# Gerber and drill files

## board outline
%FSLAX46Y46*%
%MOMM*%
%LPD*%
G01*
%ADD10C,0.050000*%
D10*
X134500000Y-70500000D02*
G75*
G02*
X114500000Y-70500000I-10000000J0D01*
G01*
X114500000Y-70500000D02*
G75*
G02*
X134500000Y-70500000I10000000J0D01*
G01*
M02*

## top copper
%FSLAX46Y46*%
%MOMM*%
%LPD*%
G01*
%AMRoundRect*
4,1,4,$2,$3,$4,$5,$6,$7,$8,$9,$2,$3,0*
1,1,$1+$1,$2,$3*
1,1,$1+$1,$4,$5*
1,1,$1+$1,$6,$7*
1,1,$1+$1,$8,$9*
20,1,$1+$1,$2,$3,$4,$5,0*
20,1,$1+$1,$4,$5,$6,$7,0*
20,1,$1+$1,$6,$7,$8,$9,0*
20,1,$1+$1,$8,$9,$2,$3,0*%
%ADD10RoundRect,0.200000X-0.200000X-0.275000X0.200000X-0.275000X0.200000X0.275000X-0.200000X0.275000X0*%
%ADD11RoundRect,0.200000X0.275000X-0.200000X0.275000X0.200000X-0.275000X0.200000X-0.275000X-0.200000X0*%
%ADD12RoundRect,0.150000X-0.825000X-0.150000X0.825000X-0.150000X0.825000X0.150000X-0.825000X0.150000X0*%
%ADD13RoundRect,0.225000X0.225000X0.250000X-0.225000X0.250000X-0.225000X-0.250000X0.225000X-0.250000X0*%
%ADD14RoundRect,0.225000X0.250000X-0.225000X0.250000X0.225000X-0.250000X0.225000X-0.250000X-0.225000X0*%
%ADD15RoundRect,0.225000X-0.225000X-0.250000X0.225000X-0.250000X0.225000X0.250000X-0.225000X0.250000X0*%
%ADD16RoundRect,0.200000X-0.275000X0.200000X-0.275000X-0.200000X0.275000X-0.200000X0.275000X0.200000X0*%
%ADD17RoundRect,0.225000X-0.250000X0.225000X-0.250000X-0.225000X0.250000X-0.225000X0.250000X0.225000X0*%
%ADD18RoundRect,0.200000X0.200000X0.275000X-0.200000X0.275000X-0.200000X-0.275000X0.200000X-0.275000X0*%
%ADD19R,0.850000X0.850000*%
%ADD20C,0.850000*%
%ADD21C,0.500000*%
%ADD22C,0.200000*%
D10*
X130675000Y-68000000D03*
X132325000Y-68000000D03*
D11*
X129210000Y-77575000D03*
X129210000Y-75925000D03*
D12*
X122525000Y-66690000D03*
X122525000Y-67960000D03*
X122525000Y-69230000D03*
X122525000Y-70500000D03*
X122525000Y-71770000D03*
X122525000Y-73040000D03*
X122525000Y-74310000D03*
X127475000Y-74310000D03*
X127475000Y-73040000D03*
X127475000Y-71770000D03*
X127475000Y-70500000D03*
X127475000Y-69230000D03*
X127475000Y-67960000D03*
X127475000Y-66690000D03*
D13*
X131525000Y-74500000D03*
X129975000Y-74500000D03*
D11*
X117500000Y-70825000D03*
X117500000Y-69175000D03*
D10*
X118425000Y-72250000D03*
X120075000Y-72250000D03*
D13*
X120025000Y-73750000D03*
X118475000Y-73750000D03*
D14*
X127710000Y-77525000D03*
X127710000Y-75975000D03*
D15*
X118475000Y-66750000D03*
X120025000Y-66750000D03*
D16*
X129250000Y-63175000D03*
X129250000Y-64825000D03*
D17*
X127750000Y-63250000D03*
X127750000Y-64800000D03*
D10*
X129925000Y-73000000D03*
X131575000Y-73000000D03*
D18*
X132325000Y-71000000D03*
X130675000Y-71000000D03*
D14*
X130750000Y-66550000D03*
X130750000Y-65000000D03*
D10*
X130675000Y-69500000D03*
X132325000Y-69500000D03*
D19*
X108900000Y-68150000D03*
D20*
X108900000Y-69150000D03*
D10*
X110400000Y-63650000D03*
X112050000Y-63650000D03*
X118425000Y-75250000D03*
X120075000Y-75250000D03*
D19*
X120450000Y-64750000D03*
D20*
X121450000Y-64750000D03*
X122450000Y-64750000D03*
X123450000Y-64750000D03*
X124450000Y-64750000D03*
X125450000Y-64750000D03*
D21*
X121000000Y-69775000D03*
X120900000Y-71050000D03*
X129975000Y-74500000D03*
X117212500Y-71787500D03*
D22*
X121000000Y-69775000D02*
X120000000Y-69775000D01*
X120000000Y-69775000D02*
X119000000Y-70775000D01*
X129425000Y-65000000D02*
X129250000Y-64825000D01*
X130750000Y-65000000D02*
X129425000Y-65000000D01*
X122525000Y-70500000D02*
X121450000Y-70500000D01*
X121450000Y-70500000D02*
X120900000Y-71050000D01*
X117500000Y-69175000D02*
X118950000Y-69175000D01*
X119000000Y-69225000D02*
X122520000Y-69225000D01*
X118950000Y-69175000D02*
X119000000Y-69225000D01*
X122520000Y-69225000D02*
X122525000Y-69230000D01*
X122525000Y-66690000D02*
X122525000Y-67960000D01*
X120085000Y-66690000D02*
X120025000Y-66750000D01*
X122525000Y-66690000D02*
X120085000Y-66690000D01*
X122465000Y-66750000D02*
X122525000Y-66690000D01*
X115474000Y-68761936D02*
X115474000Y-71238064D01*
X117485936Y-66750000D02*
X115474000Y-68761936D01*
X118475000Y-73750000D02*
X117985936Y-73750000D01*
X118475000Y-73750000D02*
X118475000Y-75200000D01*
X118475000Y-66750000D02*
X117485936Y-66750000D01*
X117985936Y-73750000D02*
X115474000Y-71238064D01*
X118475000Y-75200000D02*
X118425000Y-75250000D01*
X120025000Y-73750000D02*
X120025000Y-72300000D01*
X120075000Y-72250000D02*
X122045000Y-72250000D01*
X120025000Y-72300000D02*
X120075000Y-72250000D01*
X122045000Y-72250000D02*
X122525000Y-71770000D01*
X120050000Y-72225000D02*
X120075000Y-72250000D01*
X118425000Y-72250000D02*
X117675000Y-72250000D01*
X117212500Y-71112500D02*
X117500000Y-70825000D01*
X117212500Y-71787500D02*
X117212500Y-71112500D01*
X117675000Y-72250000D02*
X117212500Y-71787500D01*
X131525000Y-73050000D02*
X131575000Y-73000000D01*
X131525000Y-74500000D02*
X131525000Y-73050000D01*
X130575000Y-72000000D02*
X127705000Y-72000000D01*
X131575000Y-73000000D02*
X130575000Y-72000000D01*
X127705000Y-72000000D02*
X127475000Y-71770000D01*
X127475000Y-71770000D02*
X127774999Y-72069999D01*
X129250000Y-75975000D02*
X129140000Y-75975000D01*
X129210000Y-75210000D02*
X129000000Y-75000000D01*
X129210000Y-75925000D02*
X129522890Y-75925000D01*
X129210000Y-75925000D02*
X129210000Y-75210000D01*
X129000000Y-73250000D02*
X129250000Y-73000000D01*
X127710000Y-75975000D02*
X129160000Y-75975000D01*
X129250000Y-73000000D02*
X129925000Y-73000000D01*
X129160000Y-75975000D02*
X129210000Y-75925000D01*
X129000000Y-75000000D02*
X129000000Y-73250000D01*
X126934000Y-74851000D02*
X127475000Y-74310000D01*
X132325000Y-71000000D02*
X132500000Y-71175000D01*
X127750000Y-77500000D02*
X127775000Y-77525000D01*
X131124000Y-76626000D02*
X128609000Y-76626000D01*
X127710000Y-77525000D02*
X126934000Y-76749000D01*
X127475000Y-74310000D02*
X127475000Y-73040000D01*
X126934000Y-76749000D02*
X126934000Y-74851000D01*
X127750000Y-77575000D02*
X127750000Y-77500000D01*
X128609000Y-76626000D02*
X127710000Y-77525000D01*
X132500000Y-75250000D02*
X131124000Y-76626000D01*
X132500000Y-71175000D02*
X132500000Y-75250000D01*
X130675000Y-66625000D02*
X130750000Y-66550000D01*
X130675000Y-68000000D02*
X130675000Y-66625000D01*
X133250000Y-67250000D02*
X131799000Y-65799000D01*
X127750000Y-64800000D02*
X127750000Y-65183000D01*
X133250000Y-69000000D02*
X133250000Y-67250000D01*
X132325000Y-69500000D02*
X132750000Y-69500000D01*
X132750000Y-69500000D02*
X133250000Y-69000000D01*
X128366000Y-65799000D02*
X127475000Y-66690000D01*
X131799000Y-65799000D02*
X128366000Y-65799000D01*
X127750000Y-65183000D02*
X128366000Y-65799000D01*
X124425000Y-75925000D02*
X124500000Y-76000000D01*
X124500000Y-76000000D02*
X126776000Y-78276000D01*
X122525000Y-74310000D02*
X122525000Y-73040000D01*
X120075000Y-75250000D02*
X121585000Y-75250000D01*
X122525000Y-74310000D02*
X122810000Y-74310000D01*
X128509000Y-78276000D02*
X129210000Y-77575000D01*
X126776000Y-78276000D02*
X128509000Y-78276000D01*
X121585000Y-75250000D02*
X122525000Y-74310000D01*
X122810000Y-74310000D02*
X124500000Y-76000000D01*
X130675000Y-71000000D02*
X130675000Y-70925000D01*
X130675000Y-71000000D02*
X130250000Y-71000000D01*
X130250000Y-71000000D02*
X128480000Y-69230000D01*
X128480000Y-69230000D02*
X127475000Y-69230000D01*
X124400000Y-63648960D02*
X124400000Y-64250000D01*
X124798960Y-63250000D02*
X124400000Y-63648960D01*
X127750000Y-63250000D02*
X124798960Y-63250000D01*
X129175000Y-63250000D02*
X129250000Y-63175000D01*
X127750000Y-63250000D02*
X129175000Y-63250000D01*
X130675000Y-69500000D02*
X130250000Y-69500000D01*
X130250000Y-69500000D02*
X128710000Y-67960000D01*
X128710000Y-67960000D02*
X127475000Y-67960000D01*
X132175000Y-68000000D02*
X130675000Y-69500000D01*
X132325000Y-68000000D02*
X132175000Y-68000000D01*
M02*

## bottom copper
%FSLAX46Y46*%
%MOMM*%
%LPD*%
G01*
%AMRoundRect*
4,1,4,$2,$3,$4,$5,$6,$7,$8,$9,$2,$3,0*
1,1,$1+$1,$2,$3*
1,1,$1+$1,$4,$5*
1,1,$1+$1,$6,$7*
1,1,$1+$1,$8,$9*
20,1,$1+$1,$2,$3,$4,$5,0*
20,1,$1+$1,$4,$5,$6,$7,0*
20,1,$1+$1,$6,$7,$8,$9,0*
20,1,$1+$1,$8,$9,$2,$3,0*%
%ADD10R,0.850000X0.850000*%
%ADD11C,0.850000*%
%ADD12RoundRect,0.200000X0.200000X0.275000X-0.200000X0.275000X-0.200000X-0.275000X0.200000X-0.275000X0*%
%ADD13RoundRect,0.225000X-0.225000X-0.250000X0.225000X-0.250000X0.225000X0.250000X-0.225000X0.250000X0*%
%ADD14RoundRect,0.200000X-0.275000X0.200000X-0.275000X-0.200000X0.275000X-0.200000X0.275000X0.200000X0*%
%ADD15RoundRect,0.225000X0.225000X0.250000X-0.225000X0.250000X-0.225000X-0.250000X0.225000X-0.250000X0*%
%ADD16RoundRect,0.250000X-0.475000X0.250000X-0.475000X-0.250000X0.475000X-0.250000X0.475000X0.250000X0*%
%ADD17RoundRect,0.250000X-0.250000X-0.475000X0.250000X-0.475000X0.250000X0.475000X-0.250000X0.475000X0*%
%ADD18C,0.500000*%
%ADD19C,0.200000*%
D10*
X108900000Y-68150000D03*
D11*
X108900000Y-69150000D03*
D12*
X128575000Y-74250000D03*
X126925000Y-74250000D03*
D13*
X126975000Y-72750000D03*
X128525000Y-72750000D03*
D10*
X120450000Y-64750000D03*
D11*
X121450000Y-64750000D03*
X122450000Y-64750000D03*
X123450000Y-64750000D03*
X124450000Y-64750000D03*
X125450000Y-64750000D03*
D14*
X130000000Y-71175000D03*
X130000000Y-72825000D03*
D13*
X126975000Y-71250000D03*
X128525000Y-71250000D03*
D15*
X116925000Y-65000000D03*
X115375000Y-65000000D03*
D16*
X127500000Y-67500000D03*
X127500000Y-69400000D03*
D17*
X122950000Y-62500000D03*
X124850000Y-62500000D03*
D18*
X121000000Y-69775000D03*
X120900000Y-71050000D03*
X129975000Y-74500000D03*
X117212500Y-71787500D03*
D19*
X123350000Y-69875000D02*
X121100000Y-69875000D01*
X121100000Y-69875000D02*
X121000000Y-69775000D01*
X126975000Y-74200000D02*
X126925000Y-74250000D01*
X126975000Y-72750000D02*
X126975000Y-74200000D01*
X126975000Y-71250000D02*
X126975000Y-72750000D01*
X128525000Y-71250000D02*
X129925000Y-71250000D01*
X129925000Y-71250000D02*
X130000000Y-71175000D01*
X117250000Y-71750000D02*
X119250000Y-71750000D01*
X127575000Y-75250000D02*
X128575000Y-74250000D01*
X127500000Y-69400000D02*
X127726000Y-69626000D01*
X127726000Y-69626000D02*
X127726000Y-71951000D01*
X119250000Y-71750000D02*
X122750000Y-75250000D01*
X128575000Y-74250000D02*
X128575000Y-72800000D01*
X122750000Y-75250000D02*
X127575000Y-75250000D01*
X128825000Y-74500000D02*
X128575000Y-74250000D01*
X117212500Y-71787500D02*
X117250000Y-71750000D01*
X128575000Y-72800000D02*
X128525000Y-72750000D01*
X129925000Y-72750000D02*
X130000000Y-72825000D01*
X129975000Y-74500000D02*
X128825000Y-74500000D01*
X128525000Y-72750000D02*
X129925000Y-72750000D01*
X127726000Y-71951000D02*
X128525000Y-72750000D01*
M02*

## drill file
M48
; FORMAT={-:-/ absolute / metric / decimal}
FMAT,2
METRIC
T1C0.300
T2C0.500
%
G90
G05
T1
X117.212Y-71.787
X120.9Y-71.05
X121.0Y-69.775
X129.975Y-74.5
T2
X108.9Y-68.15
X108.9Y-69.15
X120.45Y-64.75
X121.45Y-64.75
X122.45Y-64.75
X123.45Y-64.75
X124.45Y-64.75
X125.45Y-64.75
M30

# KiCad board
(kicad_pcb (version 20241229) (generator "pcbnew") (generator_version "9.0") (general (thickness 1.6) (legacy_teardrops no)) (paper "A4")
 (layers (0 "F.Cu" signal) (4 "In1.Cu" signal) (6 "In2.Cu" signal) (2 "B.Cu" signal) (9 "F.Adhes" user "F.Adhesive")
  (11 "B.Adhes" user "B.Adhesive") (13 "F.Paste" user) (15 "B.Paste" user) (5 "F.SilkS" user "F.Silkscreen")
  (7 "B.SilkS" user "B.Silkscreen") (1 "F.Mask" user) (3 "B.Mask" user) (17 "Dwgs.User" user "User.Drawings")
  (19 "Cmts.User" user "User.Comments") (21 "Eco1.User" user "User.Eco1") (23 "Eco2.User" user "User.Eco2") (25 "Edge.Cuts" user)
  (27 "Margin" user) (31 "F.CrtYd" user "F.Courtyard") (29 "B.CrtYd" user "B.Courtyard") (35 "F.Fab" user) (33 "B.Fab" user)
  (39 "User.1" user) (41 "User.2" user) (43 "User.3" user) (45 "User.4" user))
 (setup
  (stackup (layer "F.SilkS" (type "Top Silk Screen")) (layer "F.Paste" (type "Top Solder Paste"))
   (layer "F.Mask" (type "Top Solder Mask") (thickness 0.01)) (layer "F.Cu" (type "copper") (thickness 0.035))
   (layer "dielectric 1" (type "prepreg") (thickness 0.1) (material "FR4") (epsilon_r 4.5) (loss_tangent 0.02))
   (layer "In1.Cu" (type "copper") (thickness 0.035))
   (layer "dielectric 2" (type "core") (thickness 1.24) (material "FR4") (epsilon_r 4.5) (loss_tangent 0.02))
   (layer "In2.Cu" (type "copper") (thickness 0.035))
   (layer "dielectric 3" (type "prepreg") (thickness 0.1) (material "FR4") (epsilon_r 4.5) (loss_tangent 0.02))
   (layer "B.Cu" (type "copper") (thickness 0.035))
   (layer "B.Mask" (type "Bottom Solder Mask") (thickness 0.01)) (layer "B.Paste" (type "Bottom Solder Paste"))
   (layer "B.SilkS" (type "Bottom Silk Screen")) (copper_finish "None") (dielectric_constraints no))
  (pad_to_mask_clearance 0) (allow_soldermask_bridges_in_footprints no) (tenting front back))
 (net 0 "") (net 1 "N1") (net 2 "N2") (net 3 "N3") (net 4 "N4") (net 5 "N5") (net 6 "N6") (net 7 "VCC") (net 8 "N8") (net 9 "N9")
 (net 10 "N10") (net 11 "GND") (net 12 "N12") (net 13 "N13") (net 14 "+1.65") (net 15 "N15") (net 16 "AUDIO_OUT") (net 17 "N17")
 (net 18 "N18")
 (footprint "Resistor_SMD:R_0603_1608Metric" (layer "F.Cu") (at 131.5 68)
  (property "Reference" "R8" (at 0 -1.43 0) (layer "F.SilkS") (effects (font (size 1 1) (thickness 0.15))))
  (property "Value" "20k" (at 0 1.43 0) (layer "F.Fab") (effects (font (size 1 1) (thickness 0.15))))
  (pad "1" smd roundrect (at -0.825 0) (size 0.8 0.95) (layers "F.Cu" "F.Mask" "F.Paste") (roundrect_rratio 0.25) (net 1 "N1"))
  (pad "2" smd roundrect (at 0.825 0) (size 0.8 0.95) (layers "F.Cu" "F.Mask" "F.Paste") (roundrect_rratio 0.25) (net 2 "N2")))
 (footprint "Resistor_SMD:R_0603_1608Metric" (layer "F.Cu") (at 129.21 76.75 90)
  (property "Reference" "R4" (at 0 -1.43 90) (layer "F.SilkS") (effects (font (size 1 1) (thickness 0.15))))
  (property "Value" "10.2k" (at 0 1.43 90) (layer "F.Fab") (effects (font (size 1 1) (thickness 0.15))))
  (pad "1" smd roundrect (at -0.825 0 90) (size 0.8 0.95) (layers "F.Cu" "F.Mask" "F.Paste") (roundrect_rratio 0.25) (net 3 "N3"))
  (pad "2" smd roundrect (at 0.825 0 90) (size 0.8 0.95) (layers "F.Cu" "F.Mask" "F.Paste") (roundrect_rratio 0.25) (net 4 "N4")))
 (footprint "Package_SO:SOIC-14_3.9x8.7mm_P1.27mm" (layer "F.Cu") (at 125 70.5)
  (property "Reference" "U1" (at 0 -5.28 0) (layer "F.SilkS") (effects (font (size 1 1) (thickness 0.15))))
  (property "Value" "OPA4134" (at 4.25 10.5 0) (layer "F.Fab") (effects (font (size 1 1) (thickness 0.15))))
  (pad "1" smd roundrect (at -2.475 -3.81) (size 1.95 0.6) (layers "F.Cu" "F.Mask" "F.Paste") (roundrect_rratio 0.25) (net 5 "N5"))
  (pad "2" smd roundrect (at -2.475 -2.54) (size 1.95 0.6) (layers "F.Cu" "F.Mask" "F.Paste") (roundrect_rratio 0.25) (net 5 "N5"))
  (pad "3" smd roundrect (at -2.475 -1.27) (size 1.95 0.6) (layers "F.Cu" "F.Mask" "F.Paste") (roundrect_rratio 0.25) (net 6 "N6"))
  (pad "4" smd roundrect (at -2.475 0) (size 1.95 0.6) (layers "F.Cu" "F.Mask" "F.Paste") (roundrect_rratio 0.25) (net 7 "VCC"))
  (pad "5" smd roundrect (at -2.475 1.27) (size 1.95 0.6) (layers "F.Cu" "F.Mask" "F.Paste") (roundrect_rratio 0.25) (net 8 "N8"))
  (pad "6" smd roundrect (at -2.475 2.54) (size 1.95 0.6) (layers "F.Cu" "F.Mask" "F.Paste") (roundrect_rratio 0.25) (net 3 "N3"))
  (pad "7" smd roundrect (at -2.475 3.81) (size 1.95 0.6) (layers "F.Cu" "F.Mask" "F.Paste") (roundrect_rratio 0.25) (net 3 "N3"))
  (pad "8" smd roundrect (at 2.475 3.81) (size 1.95 0.6) (layers "F.Cu" "F.Mask" "F.Paste") (roundrect_rratio 0.25) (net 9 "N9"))
  (pad "9" smd roundrect (at 2.475 2.54) (size 1.95 0.6) (layers "F.Cu" "F.Mask" "F.Paste") (roundrect_rratio 0.25) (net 9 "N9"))
  (pad "10" smd roundrect (at 2.475 1.27) (size 1.95 0.6) (layers "F.Cu" "F.Mask" "F.Paste") (roundrect_rratio 0.25) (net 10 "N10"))
  (pad "11" smd roundrect (at 2.475 0) (size 1.95 0.6) (layers "F.Cu" "F.Mask" "F.Paste") (roundrect_rratio 0.25) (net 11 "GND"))
  (pad "12" smd roundrect (at 2.475 -1.27) (size 1.95 0.6) (layers "F.Cu" "F.Mask" "F.Paste") (roundrect_rratio 0.25) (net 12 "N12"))
  (pad "13" smd roundrect (at 2.475 -2.54) (size 1.95 0.6) (layers "F.Cu" "F.Mask" "F.Paste") (roundrect_rratio 0.25) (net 2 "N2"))
  (pad "14" smd roundrect (at 2.475 -3.81) (size 1.95 0.6) (layers "F.Cu" "F.Mask" "F.Paste") (roundrect_rratio 0.25) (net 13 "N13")))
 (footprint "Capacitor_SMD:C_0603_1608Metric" (layer "F.Cu") (at 130.75 74.5 180)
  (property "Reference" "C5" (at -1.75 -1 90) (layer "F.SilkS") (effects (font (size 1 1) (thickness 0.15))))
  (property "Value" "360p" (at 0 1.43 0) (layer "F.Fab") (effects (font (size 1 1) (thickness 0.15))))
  (pad "1" smd roundrect (at -0.775 0 180) (size 0.9 0.95) (layers "F.Cu" "F.Mask" "F.Paste") (roundrect_rratio 0.25) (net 10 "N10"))
  (pad "2" smd roundrect (at 0.775 0 180) (size 0.9 0.95) (layers "F.Cu" "F.Mask" "F.Paste") (roundrect_rratio 0.25) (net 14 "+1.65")))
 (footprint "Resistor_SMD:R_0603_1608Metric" (layer "F.Cu") (at 117.5 70 90)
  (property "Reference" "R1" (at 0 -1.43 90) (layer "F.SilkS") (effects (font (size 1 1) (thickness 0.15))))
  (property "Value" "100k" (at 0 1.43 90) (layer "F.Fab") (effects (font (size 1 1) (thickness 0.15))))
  (pad "1" smd roundrect (at -0.825 0 90) (size 0.8 0.95) (layers "F.Cu" "F.Mask" "F.Paste") (roundrect_rratio 0.25) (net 14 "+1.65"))
  (pad "2" smd roundrect (at 0.825 0 90) (size 0.8 0.95) (layers "F.Cu" "F.Mask" "F.Paste") (roundrect_rratio 0.25) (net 6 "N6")))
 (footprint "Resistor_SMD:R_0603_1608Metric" (layer "F.Cu") (at 119.25 72.25)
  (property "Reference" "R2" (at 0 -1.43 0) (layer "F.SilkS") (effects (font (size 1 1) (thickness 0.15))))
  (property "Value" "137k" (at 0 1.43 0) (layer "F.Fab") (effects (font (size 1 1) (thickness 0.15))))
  (pad "1" smd roundrect (at -0.825 0) (size 0.8 0.95) (layers "F.Cu" "F.Mask" "F.Paste") (roundrect_rratio 0.25) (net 14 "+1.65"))
  (pad "2" smd roundrect (at 0.825 0) (size 0.8 0.95) (layers "F.Cu" "F.Mask" "F.Paste") (roundrect_rratio 0.25) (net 8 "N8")))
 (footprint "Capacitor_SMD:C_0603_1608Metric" (layer "F.Cu") (at 119.25 73.75 180)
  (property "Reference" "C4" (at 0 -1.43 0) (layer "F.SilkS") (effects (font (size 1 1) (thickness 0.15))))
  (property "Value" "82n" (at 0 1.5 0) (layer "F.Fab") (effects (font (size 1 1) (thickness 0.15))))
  (pad "1" smd roundrect (at -0.775 0 180) (size 0.9 0.95) (layers "F.Cu" "F.Mask" "F.Paste") (roundrect_rratio 0.25) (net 8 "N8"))
  (pad "2" smd roundrect (at 0.775 0 180) (size 0.9 0.95) (layers "F.Cu" "F.Mask" "F.Paste") (roundrect_rratio 0.25) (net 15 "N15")))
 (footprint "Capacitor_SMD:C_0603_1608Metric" (layer "F.Cu") (at 127.71 76.75 90)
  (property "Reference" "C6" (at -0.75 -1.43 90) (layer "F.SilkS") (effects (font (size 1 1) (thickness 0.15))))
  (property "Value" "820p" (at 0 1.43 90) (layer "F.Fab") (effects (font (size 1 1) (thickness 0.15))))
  (pad "1" smd roundrect (at -0.775 0 90) (size 0.9 0.95) (layers "F.Cu" "F.Mask" "F.Paste") (roundrect_rratio 0.25) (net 9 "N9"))
  (pad "2" smd roundrect (at 0.775 0 90) (size 0.9 0.95) (layers "F.Cu" "F.Mask" "F.Paste") (roundrect_rratio 0.25) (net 4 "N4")))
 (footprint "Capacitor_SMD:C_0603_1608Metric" (layer "F.Cu") (at 119.25 66.75)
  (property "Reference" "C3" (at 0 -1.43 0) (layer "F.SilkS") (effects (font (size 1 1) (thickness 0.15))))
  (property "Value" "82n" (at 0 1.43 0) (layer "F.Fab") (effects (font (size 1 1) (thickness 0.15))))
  (pad "1" smd roundrect (at -0.775 0) (size 0.9 0.95) (layers "F.Cu" "F.Mask" "F.Paste") (roundrect_rratio 0.25) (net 15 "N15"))
  (pad "2" smd roundrect (at 0.775 0) (size 0.9 0.95) (layers "F.Cu" "F.Mask" "F.Paste") (roundrect_rratio 0.25) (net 5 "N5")))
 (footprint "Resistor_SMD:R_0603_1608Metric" (layer "F.Cu") (at 129.25 64 -90)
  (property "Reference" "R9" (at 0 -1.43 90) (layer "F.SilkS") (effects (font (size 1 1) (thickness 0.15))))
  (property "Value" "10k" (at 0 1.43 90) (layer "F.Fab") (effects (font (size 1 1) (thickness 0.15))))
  (pad "1" smd roundrect (at -0.825 0 270) (size 0.8 0.95) (layers "F.Cu" "F.Mask" "F.Paste") (roundrect_rratio 0.25) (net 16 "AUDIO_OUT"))
  (pad "2" smd roundrect (at 0.825 0 270) (size 0.8 0.95) (layers "F.Cu" "F.Mask" "F.Paste") (roundrect_rratio 0.25) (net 11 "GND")))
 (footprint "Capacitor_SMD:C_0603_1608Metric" (layer "F.Cu") (at 127.75 64.025 -90)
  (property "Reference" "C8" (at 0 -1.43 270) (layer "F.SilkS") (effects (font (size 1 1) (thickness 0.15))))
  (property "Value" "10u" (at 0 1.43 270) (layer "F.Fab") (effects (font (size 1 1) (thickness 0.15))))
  (pad "1" smd roundrect (at -0.775 0 270) (size 0.9 0.95) (layers "F.Cu" "F.Mask" "F.Paste") (roundrect_rratio 0.25) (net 16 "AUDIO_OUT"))
  (pad "2" smd roundrect (at 0.775 0 270) (size 0.9 0.95) (layers "F.Cu" "F.Mask" "F.Paste") (roundrect_rratio 0.25) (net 13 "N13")))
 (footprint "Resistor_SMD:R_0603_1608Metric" (layer "F.Cu") (at 130.75 73)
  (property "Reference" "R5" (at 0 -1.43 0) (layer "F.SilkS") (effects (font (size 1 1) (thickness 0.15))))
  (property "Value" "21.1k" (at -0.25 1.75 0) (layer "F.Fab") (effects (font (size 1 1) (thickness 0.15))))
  (pad "1" smd roundrect (at -0.825 0) (size 0.8 0.95) (layers "F.Cu" "F.Mask" "F.Paste") (roundrect_rratio 0.25) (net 4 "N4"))
  (pad "2" smd roundrect (at 0.825 0) (size 0.8 0.95) (layers "F.Cu" "F.Mask" "F.Paste") (roundrect_rratio 0.25) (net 10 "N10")))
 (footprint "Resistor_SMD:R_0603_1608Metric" (layer "F.Cu") (at 131.5 71 180)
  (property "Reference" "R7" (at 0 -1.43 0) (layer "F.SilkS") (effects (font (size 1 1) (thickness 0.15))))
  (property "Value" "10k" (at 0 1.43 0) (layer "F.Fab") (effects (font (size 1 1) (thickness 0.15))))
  (pad "1" smd roundrect (at -0.825 0 180) (size 0.8 0.95) (layers "F.Cu" "F.Mask" "F.Paste") (roundrect_rratio 0.25) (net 9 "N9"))
  (pad "2" smd roundrect (at 0.825 0 180) (size 0.8 0.95) (layers "F.Cu" "F.Mask" "F.Paste") (roundrect_rratio 0.25) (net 12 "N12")))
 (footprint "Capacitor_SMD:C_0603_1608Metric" (layer "F.Cu") (at 130.75 65.775 90)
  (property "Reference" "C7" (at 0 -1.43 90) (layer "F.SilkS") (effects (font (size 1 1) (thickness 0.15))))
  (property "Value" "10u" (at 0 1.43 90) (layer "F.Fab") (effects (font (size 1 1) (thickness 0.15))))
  (pad "1" smd roundrect (at -0.775 0 90) (size 0.9 0.95) (layers "F.Cu" "F.Mask" "F.Paste") (roundrect_rratio 0.25) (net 1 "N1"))
  (pad "2" smd roundrect (at 0.775 0 90) (size 0.9 0.95) (layers "F.Cu" "F.Mask" "F.Paste") (roundrect_rratio 0.25) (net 11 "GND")))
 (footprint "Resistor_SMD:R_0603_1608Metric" (layer "F.Cu") (at 131.5 69.5)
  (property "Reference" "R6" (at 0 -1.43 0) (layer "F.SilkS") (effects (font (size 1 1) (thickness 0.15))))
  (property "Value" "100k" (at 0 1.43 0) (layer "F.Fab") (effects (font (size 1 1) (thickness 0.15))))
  (pad "1" smd roundrect (at -0.825 0) (size 0.8 0.95) (layers "F.Cu" "F.Mask" "F.Paste") (roundrect_rratio 0.25) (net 2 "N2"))
  (pad "2" smd roundrect (at 0.825 0) (size 0.8 0.95) (layers "F.Cu" "F.Mask" "F.Paste") (roundrect_rratio 0.25) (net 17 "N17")))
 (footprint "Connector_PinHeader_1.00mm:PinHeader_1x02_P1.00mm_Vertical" (layer "F.Cu") (at 108.9 68.15)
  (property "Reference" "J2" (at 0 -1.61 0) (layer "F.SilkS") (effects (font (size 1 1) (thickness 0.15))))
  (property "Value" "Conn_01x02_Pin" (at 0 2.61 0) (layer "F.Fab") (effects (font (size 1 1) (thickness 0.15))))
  (pad "1" thru_hole rect (at 0 0) (size 0.85 0.85) (drill 0.5) (layers "*.Cu" "*.Mask") (remove_unused_layers no) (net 2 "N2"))
  (pad "2" thru_hole circle (at 0 1) (size 0.85 0.85) (drill 0.5) (layers "*.Cu" "*.Mask") (remove_unused_layers no) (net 17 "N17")))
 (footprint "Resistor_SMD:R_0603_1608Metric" (layer "F.Cu") (at 111.225 63.65)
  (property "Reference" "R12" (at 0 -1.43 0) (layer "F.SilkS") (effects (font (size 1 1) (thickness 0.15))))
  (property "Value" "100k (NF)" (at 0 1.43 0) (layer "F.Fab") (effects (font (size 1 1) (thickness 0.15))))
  (pad "1" smd roundrect (at -0.825 0) (size 0.8 0.95) (layers "F.Cu" "F.Mask" "F.Paste") (roundrect_rratio 0.25) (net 17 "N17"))
  (pad "2" smd roundrect (at 0.825 0) (size 0.8 0.95) (layers "F.Cu" "F.Mask" "F.Paste") (roundrect_rratio 0.25) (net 13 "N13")))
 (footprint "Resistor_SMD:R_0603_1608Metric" (layer "F.Cu") (at 119.25 75.25)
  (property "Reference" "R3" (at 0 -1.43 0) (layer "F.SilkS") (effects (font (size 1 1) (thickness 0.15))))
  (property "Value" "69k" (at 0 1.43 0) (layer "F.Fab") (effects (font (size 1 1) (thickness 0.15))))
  (pad "1" smd roundrect (at -0.825 0) (size 0.8 0.95) (layers "F.Cu" "F.Mask" "F.Paste") (roundrect_rratio 0.25) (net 15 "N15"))
  (pad "2" smd roundrect (at 0.825 0) (size 0.8 0.95) (layers "F.Cu" "F.Mask" "F.Paste") (roundrect_rratio 0.25) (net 3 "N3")))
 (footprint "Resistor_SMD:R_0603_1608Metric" (layer "B.Cu") (at 127.75 74.25 180)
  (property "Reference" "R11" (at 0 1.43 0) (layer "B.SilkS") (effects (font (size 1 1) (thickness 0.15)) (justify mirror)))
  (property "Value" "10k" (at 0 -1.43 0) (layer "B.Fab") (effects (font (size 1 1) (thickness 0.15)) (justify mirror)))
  (pad "1" smd roundrect (at -0.825 0 180) (size 0.8 0.95) (layers "B.Cu" "B.Mask" "B.Paste") (roundrect_rratio 0.25) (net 14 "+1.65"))
  (pad "2" smd roundrect (at 0.825 0 180) (size 0.8 0.95) (layers "B.Cu" "B.Mask" "B.Paste") (roundrect_rratio 0.25) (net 11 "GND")))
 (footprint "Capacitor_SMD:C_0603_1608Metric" (layer "B.Cu") (at 127.75 72.75)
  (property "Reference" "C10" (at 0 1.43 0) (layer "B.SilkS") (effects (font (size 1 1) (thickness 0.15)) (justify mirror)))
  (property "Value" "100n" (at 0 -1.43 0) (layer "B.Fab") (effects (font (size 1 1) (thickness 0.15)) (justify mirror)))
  (pad "1" smd roundrect (at -0.775 0) (size 0.9 0.95) (layers "B.Cu" "B.Mask" "B.Paste") (roundrect_rratio 0.25) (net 11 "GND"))
  (pad "2" smd roundrect (at 0.775 0) (size 0.9 0.95) (layers "B.Cu" "B.Mask" "B.Paste") (roundrect_rratio 0.25) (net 14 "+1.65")))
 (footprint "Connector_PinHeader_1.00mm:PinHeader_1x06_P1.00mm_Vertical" (layer "B.Cu") (at 120.45 64.75 -90)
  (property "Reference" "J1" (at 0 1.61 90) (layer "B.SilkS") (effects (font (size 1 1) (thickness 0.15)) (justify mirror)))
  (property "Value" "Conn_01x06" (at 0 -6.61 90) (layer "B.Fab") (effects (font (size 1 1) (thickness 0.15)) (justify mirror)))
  (pad "1" thru_hole rect (at 0 0 270) (size 0.85 0.85) (drill 0.5) (layers "*.Cu" "*.Mask") (remove_unused_layers no) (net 11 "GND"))
  (pad "2" thru_hole circle (at 0 -1 270) (size 0.85 0.85) (drill 0.5) (layers "*.Cu" "*.Mask") (remove_unused_layers no) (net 11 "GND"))
  (pad "3" thru_hole circle (at 0 -2 270) (size 0.85 0.85) (drill 0.5) (layers "*.Cu" "*.Mask") (remove_unused_layers no) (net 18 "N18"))
  (pad "4" thru_hole circle (at 0 -3 270) (size 0.85 0.85) (drill 0.5) (layers "*.Cu" "*.Mask") (remove_unused_layers no) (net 11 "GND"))
  (pad "5" thru_hole circle (at 0 -4 270) (size 0.85 0.85) (drill 0.5) (layers "*.Cu" "*.Mask") (remove_unused_layers no)
   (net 16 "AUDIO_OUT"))
  (pad "6" thru_hole circle (at 0 -5 270) (size 0.85 0.85) (drill 0.5) (layers "*.Cu" "*.Mask") (remove_unused_layers no) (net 7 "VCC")))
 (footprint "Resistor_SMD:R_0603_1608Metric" (layer "B.Cu") (at 130 72 -90)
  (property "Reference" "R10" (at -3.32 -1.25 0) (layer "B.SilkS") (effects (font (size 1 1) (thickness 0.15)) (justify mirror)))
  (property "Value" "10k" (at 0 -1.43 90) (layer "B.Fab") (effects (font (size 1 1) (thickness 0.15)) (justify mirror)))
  (pad "1" smd roundrect (at -0.825 0 270) (size 0.8 0.95) (layers "B.Cu" "B.Mask" "B.Paste") (roundrect_rratio 0.25) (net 7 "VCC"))
  (pad "2" smd roundrect (at 0.825 0 270) (size 0.8 0.95) (layers "B.Cu" "B.Mask" "B.Paste") (roundrect_rratio 0.25) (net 14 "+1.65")))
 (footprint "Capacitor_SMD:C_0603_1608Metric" (layer "B.Cu") (at 127.75 71.25)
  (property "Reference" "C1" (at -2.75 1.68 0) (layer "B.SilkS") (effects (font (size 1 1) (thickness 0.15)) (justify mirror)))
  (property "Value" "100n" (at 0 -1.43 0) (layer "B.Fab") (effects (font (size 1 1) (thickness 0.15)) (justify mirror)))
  (pad "1" smd roundrect (at -0.775 0) (size 0.9 0.95) (layers "B.Cu" "B.Mask" "B.Paste") (roundrect_rratio 0.25) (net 11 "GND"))
  (pad "2" smd roundrect (at 0.775 0) (size 0.9 0.95) (layers "B.Cu" "B.Mask" "B.Paste") (roundrect_rratio 0.25) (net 7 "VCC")))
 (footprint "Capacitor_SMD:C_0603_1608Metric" (layer "B.Cu") (at 116.15 65 180)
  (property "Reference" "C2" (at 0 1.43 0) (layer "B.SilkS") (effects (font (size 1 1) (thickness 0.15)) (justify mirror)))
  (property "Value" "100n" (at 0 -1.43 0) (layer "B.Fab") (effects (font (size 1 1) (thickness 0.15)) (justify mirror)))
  (pad "1" smd roundrect (at -0.775 0 180) (size 0.9 0.95) (layers "B.Cu" "B.Mask" "B.Paste") (roundrect_rratio 0.25) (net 6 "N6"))
  (pad "2" smd roundrect (at 0.775 0 180) (size 0.9 0.95) (layers "B.Cu" "B.Mask" "B.Paste") (roundrect_rratio 0.25) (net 18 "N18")))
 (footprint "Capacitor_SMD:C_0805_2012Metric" (layer "B.Cu") (at 127.5 68.45 -90)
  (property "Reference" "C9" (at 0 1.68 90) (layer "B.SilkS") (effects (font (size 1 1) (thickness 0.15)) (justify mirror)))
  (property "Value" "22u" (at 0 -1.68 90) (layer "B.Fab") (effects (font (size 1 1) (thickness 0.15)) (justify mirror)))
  (pad "1" smd roundrect (at -0.95 0 270) (size 1 1.45) (layers "B.Cu" "B.Mask" "B.Paste") (roundrect_rratio 0.25) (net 11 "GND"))
  (pad "2" smd roundrect (at 0.95 0 270) (size 1 1.45) (layers "B.Cu" "B.Mask" "B.Paste") (roundrect_rratio 0.25) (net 14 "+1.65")))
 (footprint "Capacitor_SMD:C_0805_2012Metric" (layer "B.Cu") (at 123.9 62.5)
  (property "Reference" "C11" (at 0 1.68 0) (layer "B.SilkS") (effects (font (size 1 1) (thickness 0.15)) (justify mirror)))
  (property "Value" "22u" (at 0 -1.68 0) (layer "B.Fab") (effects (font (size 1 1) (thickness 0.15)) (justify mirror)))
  (pad "1" smd roundrect (at -0.95 0) (size 1 1.45) (layers "B.Cu" "B.Mask" "B.Paste") (roundrect_rratio 0.25) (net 11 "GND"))
  (pad "2" smd roundrect (at 0.95 0) (size 1 1.45) (layers "B.Cu" "B.Mask" "B.Paste") (roundrect_rratio 0.25) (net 7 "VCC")))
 (gr_circle (center 124.5 70.5) (end 134.5 70.5) (stroke (width 0.05) (type solid)) (fill no) (locked yes) (layer "Edge.Cuts"))
 (segment (start 121 69.775) (end 120 69.775) (width 0.2) (layer "F.Cu") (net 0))
 (segment (start 120 69.775) (end 119 70.775) (width 0.2) (layer "F.Cu") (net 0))
 (via (at 121 69.775) (size 0.5) (drill 0.3) (layers "F.Cu" "B.Cu") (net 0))
 (segment (start 123.35 69.875) (end 121.1 69.875) (width 0.2) (layer "B.Cu") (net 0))
 (segment (start 121.1 69.875) (end 121 69.775) (width 0.2) (layer "B.Cu") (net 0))
 (segment (start 129.425 65) (end 129.25 64.825) (width 0.2) (layer "F.Cu") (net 11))
 (segment (start 130.75 65) (end 129.425 65) (width 0.2) (layer "F.Cu") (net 11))
 (segment (start 126.975 74.2) (end 126.925 74.25) (width 0.2) (layer "B.Cu") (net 11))
 (segment (start 126.975 72.75) (end 126.975 74.2) (width 0.2) (layer "B.Cu") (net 11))
 (segment (start 126.975 71.25) (end 126.975 72.75) (width 0.2) (layer "B.Cu") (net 11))
 (segment (start 122.525 70.5) (end 121.45 70.5) (width 0.2) (layer "F.Cu") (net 7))
 (segment (start 121.45 70.5) (end 120.9 71.05) (width 0.2) (layer "F.Cu") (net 7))
 (via (at 120.9 71.05) (size 0.5) (drill 0.3) (layers "F.Cu" "B.Cu") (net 7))
 (segment (start 128.525 71.25) (end 129.925 71.25) (width 0.2) (layer "B.Cu") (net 7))
 (segment (start 129.925 71.25) (end 130 71.175) (width 0.2) (layer "B.Cu") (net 7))
 (segment (start 117.5 69.175) (end 118.95 69.175) (width 0.2) (layer "F.Cu") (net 6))
 (segment (start 119 69.225) (end 122.52 69.225) (width 0.2) (layer "F.Cu") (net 6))
 (segment (start 118.95 69.175) (end 119 69.225) (width 0.2) (layer "F.Cu") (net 6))
 (segment (start 122.52 69.225) (end 122.525 69.23) (width 0.2) (layer "F.Cu") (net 6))
 (segment (start 122.525 66.69) (end 122.525 67.96) (width 0.2) (layer "F.Cu") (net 5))
 (segment (start 120.085 66.69) (end 120.025 66.75) (width 0.2) (layer "F.Cu") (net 5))
 (segment (start 122.525 66.69) (end 120.085 66.69) (width 0.2) (layer "F.Cu") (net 5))
 (segment (start 122.465 66.75) (end 122.525 66.69) (width 0.2) (layer "F.Cu") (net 5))
 (segment (start 115.474 68.761936) (end 115.474 71.238064) (width 0.2) (layer "F.Cu") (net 15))
 (segment (start 117.485936 66.75) (end 115.474 68.761936) (width 0.2) (layer "F.Cu") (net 15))
 (segment (start 118.475 73.75) (end 117.985936 73.75) (width 0.2) (layer "F.Cu") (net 15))
 (segment (start 118.475 73.75) (end 118.475 75.2) (width 0.2) (layer "F.Cu") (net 15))
 (segment (start 118.475 66.75) (end 117.485936 66.75) (width 0.2) (layer "F.Cu") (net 15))
 (segment (start 117.985936 73.75) (end 115.474 71.238064) (width 0.2) (layer "F.Cu") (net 15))
 (segment (start 118.475 75.2) (end 118.425 75.25) (width 0.2) (layer "F.Cu") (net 15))
 (segment (start 120.025 73.75) (end 120.025 72.3) (width 0.2) (layer "F.Cu") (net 8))
 (segment (start 120.075 72.25) (end 122.045 72.25) (width 0.2) (layer "F.Cu") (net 8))
 (segment (start 120.025 72.3) (end 120.075 72.25) (width 0.2) (layer "F.Cu") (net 8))
 (segment (start 122.045 72.25) (end 122.525 71.77) (width 0.2) (layer "F.Cu") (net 8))
 (segment (start 120.05 72.225) (end 120.075 72.25) (width 0.2) (layer "F.Cu") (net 8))
 (segment (start 118.425 72.25) (end 117.675 72.25) (width 0.2) (layer "F.Cu") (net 14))
 (segment (start 117.2125 71.1125) (end 117.5 70.825) (width 0.2) (layer "F.Cu") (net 14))
 (segment (start 117.2125 71.7875) (end 117.2125 71.1125) (width 0.2) (layer "F.Cu") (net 14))
 (segment (start 117.675 72.25) (end 117.2125 71.7875) (width 0.2) (layer "F.Cu") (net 14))
 (via (at 129.975 74.5) (size 0.5) (drill 0.3) (layers "F.Cu" "B.Cu") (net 14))
 (via (at 117.2125 71.7875) (size 0.5) (drill 0.3) (layers "F.Cu" "B.Cu") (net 14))
 (segment (start 117.25 71.75) (end 119.25 71.75) (width 0.2) (layer "B.Cu") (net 14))
 (segment (start 127.575 75.25) (end 128.575 74.25) (width 0.2) (layer "B.Cu") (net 14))
 (segment (start 127.5 69.4) (end 127.726 69.626) (width 0.2) (layer "B.Cu") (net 14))
 (segment (start 127.726 69.626) (end 127.726 71.951) (width 0.2) (layer "B.Cu") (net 14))
 (segment (start 119.25 71.75) (end 122.75 75.25) (width 0.2) (layer "B.Cu") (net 14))
 (segment (start 128.575 74.25) (end 128.575 72.8) (width 0.2) (layer "B.Cu") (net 14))
 (segment (start 122.75 75.25) (end 127.575 75.25) (width 0.2) (layer "B.Cu") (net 14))
 (segment (start 128.825 74.5) (end 128.575 74.25) (width 0.2) (layer "B.Cu") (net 14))
 (segment (start 117.2125 71.7875) (end 117.25 71.75) (width 0.2) (layer "B.Cu") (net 14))
 (segment (start 128.575 72.8) (end 128.525 72.75) (width 0.2) (layer "B.Cu") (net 14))
 (segment (start 129.925 72.75) (end 130 72.825) (width 0.2) (layer "B.Cu") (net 14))
 (segment (start 129.975 74.5) (end 128.825 74.5) (width 0.2) (layer "B.Cu") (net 14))
 (segment (start 128.525 72.75) (end 129.925 72.75) (width 0.2) (layer "B.Cu") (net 14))
 (segment (start 127.726 71.951) (end 128.525 72.75) (width 0.2) (layer "B.Cu") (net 14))
 (segment (start 131.525 73.05) (end 131.575 73) (width 0.2) (layer "F.Cu") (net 10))
 (segment (start 131.525 74.5) (end 131.525 73.05) (width 0.2) (layer "F.Cu") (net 10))
 (segment (start 130.575 72) (end 127.705 72) (width 0.2) (layer "F.Cu") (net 10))
 (segment (start 131.575 73) (end 130.575 72) (width 0.2) (layer "F.Cu") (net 10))
 (segment (start 127.705 72) (end 127.475 71.77) (width 0.2) (layer "F.Cu") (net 10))
 (segment (start 127.475 71.77) (end 127.774999 72.069999) (width 0.2) (layer "F.Cu") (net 10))
 (segment (start 129.25 75.975) (end 129.14 75.975) (width 0.2) (layer "F.Cu") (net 4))
 (segment (start 129.21 75.21) (end 129 75) (width 0.2) (layer "F.Cu") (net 4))
 (segment (start 129.21 75.925) (end 129.52289 75.925) (width 0.2) (layer "F.Cu") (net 4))
 (segment (start 129.21 75.925) (end 129.21 75.21) (width 0.2) (layer "F.Cu") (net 4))
 (segment (start 129 73.25) (end 129.25 73) (width 0.2) (layer "F.Cu") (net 4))
 (segment (start 127.71 75.975) (end 129.16 75.975) (width 0.2) (layer "F.Cu") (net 4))
 (segment (start 129.25 73) (end 129.925 73) (width 0.2) (layer "F.Cu") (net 4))
 (segment (start 129.16 75.975) (end 129.21 75.925) (width 0.2) (layer "F.Cu") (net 4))
 (segment (start 129 75) (end 129 73.25) (width 0.2) (layer "F.Cu") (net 4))
 (segment (start 126.934 74.851) (end 127.475 74.31) (width 0.2) (layer "F.Cu") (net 9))
 (segment (start 132.325 71) (end 132.5 71.175) (width 0.2) (layer "F.Cu") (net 9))
 (segment (start 127.75 77.5) (end 127.775 77.525) (width 0.2) (layer "F.Cu") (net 9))
 (segment (start 131.124 76.626) (end 128.609 76.626) (width 0.2) (layer "F.Cu") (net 9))
 (segment (start 127.71 77.525) (end 126.934 76.749) (width 0.2) (layer "F.Cu") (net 9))
 (segment (start 127.475 74.31) (end 127.475 73.04) (width 0.2) (layer "F.Cu") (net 9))
 (segment (start 126.934 76.749) (end 126.934 74.851) (width 0.2) (layer "F.Cu") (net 9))
 (segment (start 127.75 77.575) (end 127.75 77.5) (width 0.2) (layer "F.Cu") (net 9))
 (segment (start 128.609 76.626) (end 127.71 77.525) (width 0.2) (layer "F.Cu") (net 9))
 (segment (start 132.5 75.25) (end 131.124 76.626) (width 0.2) (layer "F.Cu") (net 9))
 (segment (start 132.5 71.175) (end 132.5 75.25) (width 0.2) (layer "F.Cu") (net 9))
 (segment (start 130.675 66.625) (end 130.75 66.55) (width 0.2) (layer "F.Cu") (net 1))
 (segment (start 130.675 68) (end 130.675 66.625) (width 0.2) (layer "F.Cu") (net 1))
 (segment (start 133.25 67.25) (end 131.799 65.799) (width 0.2) (layer "F.Cu") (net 13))
 (segment (start 127.75 64.8) (end 127.75 65.183) (width 0.2) (layer "F.Cu") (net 13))
 (segment (start 133.25 69) (end 133.25 67.25) (width 0.2) (layer "F.Cu") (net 13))
 (segment (start 132.325 69.5) (end 132.75 69.5) (width 0.2) (layer "F.Cu") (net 13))
 (segment (start 132.75 69.5) (end 133.25 69) (width 0.2) (layer "F.Cu") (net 13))
 (segment (start 128.366 65.799) (end 127.475 66.69) (width 0.2) (layer "F.Cu") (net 13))
 (segment (start 131.799 65.799) (end 128.366 65.799) (width 0.2) (layer "F.Cu") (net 13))
 (segment (start 127.75 65.183) (end 128.366 65.799) (width 0.2) (layer "F.Cu") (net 13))
 (segment (start 124.425 75.925) (end 124.5 76) (width 0.2) (layer "F.Cu") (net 3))
 (segment (start 124.5 76) (end 126.776 78.276) (width 0.2) (layer "F.Cu") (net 3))
 (segment (start 122.525 74.31) (end 122.525 73.04) (width 0.2) (layer "F.Cu") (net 3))
 (segment (start 120.075 75.25) (end 121.585 75.25) (width 0.2) (layer "F.Cu") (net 3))
 (segment (start 122.525 74.31) (end 122.81 74.31) (width 0.2) (layer "F.Cu") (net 3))
 (segment (start 128.509 78.276) (end 129.21 77.575) (width 0.2) (layer "F.Cu") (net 3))
 (segment (start 126.776 78.276) (end 128.509 78.276) (width 0.2) (layer "F.Cu") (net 3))
 (segment (start 121.585 75.25) (end 122.525 74.31) (width 0.2) (layer "F.Cu") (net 3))
 (segment (start 122.81 74.31) (end 124.5 76) (width 0.2) (layer "F.Cu") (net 3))
 (segment (start 130.675 71) (end 130.675 70.925) (width 0.2) (layer "F.Cu") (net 12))
 (segment (start 130.675 71) (end 130.25 71) (width 0.2) (layer "F.Cu") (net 12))
 (segment (start 130.25 71) (end 128.48 69.23) (width 0.2) (layer "F.Cu") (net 12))
 (segment (start 128.48 69.23) (end 127.475 69.23) (width 0.2) (layer "F.Cu") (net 12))
 (segment (start 124.4 63.64896) (end 124.4 64.25) (width 0.2) (layer "F.Cu") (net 16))
 (segment (start 124.79896 63.25) (end 124.4 63.64896) (width 0.2) (layer "F.Cu") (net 16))
 (segment (start 127.75 63.25) (end 124.79896 63.25) (width 0.2) (layer "F.Cu") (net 16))
 (segment (start 129.175 63.25) (end 129.25 63.175) (width 0.2) (layer "F.Cu") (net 16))
 (segment (start 127.75 63.25) (end 129.175 63.25) (width 0.2) (layer "F.Cu") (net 16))
 (segment (start 130.675 69.5) (end 130.25 69.5) (width 0.2) (layer "F.Cu") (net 2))
 (segment (start 130.25 69.5) (end 128.71 67.96) (width 0.2) (layer "F.Cu") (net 2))
 (segment (start 128.71 67.96) (end 127.475 67.96) (width 0.2) (layer "F.Cu") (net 2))
 (segment (start 132.175 68) (end 130.675 69.5) (width 0.2) (layer "F.Cu") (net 2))
 (segment (start 132.325 68) (end 132.175 68) (width 0.2) (layer "F.Cu") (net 2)))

